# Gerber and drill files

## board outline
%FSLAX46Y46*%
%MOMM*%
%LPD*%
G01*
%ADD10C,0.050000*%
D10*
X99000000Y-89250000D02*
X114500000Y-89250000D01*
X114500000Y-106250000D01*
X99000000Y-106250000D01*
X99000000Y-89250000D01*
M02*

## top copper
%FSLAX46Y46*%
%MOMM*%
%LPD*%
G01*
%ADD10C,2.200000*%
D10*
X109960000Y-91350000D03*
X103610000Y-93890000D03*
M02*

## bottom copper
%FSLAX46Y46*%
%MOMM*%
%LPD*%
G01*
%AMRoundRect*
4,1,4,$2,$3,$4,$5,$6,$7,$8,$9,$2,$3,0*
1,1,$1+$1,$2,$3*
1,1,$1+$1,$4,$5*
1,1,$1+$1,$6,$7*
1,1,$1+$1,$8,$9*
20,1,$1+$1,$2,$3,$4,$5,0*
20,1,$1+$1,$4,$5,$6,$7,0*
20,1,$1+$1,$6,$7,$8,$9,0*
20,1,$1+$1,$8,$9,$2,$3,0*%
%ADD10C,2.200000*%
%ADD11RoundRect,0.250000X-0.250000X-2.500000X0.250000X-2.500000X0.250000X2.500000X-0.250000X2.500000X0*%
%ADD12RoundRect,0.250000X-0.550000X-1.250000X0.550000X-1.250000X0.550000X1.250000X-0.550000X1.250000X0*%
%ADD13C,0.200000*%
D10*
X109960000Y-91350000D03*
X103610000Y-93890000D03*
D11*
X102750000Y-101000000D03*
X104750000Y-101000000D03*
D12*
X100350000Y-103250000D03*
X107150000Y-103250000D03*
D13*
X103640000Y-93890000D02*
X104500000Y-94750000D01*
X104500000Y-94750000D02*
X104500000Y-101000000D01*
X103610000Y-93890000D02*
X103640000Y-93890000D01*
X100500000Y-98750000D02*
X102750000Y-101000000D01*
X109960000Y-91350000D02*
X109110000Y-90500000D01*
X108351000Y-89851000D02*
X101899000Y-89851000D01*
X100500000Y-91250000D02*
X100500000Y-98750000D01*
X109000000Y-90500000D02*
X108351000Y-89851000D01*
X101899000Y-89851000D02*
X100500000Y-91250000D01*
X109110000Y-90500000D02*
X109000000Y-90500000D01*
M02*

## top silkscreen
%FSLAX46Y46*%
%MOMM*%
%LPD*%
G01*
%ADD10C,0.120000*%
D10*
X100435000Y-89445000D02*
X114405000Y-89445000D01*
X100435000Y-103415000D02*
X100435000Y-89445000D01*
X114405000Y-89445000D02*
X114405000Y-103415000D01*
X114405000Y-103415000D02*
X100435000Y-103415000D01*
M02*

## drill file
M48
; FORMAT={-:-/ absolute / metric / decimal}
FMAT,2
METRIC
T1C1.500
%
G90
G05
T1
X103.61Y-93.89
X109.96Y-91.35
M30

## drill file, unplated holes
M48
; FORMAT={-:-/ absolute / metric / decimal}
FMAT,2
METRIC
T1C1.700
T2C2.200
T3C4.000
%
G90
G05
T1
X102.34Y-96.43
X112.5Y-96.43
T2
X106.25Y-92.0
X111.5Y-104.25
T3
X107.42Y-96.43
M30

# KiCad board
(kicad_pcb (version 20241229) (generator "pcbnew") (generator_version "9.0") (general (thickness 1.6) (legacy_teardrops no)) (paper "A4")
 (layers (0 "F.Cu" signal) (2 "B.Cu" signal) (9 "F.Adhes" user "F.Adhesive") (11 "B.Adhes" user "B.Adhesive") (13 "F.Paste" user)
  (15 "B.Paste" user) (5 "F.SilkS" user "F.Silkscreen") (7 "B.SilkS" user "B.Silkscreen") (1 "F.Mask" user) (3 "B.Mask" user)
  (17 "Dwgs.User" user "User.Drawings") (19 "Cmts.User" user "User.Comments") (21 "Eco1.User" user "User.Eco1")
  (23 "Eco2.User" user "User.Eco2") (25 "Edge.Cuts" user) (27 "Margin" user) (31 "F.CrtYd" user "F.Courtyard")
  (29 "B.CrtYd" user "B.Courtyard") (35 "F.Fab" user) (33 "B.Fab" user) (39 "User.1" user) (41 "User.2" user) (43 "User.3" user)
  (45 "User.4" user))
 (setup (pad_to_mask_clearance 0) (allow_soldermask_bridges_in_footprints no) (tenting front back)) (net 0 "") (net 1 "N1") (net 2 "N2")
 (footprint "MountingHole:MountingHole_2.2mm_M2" (layer "F.Cu") (at 111.5 104.25)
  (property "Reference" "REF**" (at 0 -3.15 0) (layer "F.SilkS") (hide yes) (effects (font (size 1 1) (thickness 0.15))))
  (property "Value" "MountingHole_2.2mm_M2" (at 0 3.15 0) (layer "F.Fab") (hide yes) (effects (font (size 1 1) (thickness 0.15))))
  (pad "" np_thru_hole circle (at 0 0) (size 2.2 2.2) (drill 2.2) (layers "*.Cu" "*.Mask")))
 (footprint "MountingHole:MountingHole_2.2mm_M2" (layer "F.Cu") (at 106.25 92)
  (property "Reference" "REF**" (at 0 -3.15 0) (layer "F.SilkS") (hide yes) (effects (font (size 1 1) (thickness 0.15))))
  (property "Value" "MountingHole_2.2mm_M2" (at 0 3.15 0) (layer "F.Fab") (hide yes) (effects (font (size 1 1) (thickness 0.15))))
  (pad "" np_thru_hole circle (at 0 0) (size 2.2 2.2) (drill 2.2) (layers "*.Cu" "*.Mask")))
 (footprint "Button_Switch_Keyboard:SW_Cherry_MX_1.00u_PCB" (layer "F.Cu") (at 109.96 91.35)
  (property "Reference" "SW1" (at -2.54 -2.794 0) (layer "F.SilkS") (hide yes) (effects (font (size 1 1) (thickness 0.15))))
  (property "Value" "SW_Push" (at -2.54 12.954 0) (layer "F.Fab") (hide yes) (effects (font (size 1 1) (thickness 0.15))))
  (fp_line (start -9.525 -1.905) (end 4.445 -1.905) (stroke (width 0.12) (type solid)) (layer "F.SilkS"))
  (fp_line (start -9.525 12.065) (end -9.525 -1.905) (stroke (width 0.12) (type solid)) (layer "F.SilkS"))
  (fp_line (start 4.445 -1.905) (end 4.445 12.065) (stroke (width 0.12) (type solid)) (layer "F.SilkS"))
  (fp_line (start 4.445 12.065) (end -9.525 12.065) (stroke (width 0.12) (type solid)) (layer "F.SilkS"))
  (pad "" np_thru_hole circle (at -7.62 5.08) (size 1.7 1.7) (drill 1.7) (layers "*.Cu" "*.Mask"))
  (pad "" np_thru_hole circle (at -2.54 5.08) (size 4 4) (drill 4) (layers "*.Cu" "*.Mask"))
  (pad "" np_thru_hole circle (at 2.54 5.08) (size 1.7 1.7) (drill 1.7) (layers "*.Cu" "*.Mask"))
  (pad "1" thru_hole circle (at 0 0) (size 2.2 2.2) (drill 1.5) (layers "*.Cu" "*.Mask") (remove_unused_layers no) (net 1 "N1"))
  (pad "2" thru_hole circle (at -6.35 2.54) (size 2.2 2.2) (drill 1.5) (layers "*.Cu" "*.Mask") (remove_unused_layers no) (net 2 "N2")))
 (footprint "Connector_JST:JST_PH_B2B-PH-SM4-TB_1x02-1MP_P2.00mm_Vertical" (layer "B.Cu") (at 103.75 101.5)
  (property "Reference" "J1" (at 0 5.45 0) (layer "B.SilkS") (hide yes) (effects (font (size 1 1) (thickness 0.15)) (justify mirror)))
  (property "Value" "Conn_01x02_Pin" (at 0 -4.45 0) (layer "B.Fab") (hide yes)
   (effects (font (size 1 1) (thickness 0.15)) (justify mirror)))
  (pad "1" smd roundrect (at -1 -0.5) (size 1 5.5) (layers "B.Cu" "B.Mask" "B.Paste") (roundrect_rratio 0.25) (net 1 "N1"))
  (pad "2" smd roundrect (at 1 -0.5) (size 1 5.5) (layers "B.Cu" "B.Mask" "B.Paste") (roundrect_rratio 0.25) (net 2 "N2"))
  (pad "MP" smd roundrect (at -3.4 1.75) (size 1.6 3) (layers "B.Cu" "B.Mask" "B.Paste") (roundrect_rratio 0.15625))
  (pad "MP" smd roundrect (at 3.4 1.75) (size 1.6 3) (layers "B.Cu" "B.Mask" "B.Paste") (roundrect_rratio 0.15625)))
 (gr_rect (start 99 89.25) (end 114.5 106.25) (stroke (width 0.05) (type default)) (fill no) (layer "Edge.Cuts"))
 (segment (start 103.64 93.89) (end 104.5 94.75) (width 0.2) (layer "B.Cu") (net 2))
 (segment (start 104.5 94.75) (end 104.5 101) (width 0.2) (layer "B.Cu") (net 2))
 (segment (start 103.61 93.89) (end 103.64 93.89) (width 0.2) (layer "B.Cu") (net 2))
 (segment (start 100.5 98.75) (end 102.75 101) (width 0.2) (layer "B.Cu") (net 1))
 (segment (start 109.96 91.35) (end 109.11 90.5) (width 0.2) (layer "B.Cu") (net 1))
 (segment (start 108.351 89.851) (end 101.899 89.851) (width 0.2) (layer "B.Cu") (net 1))
 (segment (start 100.5 91.25) (end 100.5 98.75) (width 0.2) (layer "B.Cu") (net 1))
 (segment (start 109 90.5) (end 108.351 89.851) (width 0.2) (layer "B.Cu") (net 1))
 (segment (start 101.899 89.851) (end 100.5 91.25) (width 0.2) (layer "B.Cu") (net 1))
 (segment (start 109.11 90.5) (end 109 90.5) (width 0.2) (layer "B.Cu") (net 1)))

